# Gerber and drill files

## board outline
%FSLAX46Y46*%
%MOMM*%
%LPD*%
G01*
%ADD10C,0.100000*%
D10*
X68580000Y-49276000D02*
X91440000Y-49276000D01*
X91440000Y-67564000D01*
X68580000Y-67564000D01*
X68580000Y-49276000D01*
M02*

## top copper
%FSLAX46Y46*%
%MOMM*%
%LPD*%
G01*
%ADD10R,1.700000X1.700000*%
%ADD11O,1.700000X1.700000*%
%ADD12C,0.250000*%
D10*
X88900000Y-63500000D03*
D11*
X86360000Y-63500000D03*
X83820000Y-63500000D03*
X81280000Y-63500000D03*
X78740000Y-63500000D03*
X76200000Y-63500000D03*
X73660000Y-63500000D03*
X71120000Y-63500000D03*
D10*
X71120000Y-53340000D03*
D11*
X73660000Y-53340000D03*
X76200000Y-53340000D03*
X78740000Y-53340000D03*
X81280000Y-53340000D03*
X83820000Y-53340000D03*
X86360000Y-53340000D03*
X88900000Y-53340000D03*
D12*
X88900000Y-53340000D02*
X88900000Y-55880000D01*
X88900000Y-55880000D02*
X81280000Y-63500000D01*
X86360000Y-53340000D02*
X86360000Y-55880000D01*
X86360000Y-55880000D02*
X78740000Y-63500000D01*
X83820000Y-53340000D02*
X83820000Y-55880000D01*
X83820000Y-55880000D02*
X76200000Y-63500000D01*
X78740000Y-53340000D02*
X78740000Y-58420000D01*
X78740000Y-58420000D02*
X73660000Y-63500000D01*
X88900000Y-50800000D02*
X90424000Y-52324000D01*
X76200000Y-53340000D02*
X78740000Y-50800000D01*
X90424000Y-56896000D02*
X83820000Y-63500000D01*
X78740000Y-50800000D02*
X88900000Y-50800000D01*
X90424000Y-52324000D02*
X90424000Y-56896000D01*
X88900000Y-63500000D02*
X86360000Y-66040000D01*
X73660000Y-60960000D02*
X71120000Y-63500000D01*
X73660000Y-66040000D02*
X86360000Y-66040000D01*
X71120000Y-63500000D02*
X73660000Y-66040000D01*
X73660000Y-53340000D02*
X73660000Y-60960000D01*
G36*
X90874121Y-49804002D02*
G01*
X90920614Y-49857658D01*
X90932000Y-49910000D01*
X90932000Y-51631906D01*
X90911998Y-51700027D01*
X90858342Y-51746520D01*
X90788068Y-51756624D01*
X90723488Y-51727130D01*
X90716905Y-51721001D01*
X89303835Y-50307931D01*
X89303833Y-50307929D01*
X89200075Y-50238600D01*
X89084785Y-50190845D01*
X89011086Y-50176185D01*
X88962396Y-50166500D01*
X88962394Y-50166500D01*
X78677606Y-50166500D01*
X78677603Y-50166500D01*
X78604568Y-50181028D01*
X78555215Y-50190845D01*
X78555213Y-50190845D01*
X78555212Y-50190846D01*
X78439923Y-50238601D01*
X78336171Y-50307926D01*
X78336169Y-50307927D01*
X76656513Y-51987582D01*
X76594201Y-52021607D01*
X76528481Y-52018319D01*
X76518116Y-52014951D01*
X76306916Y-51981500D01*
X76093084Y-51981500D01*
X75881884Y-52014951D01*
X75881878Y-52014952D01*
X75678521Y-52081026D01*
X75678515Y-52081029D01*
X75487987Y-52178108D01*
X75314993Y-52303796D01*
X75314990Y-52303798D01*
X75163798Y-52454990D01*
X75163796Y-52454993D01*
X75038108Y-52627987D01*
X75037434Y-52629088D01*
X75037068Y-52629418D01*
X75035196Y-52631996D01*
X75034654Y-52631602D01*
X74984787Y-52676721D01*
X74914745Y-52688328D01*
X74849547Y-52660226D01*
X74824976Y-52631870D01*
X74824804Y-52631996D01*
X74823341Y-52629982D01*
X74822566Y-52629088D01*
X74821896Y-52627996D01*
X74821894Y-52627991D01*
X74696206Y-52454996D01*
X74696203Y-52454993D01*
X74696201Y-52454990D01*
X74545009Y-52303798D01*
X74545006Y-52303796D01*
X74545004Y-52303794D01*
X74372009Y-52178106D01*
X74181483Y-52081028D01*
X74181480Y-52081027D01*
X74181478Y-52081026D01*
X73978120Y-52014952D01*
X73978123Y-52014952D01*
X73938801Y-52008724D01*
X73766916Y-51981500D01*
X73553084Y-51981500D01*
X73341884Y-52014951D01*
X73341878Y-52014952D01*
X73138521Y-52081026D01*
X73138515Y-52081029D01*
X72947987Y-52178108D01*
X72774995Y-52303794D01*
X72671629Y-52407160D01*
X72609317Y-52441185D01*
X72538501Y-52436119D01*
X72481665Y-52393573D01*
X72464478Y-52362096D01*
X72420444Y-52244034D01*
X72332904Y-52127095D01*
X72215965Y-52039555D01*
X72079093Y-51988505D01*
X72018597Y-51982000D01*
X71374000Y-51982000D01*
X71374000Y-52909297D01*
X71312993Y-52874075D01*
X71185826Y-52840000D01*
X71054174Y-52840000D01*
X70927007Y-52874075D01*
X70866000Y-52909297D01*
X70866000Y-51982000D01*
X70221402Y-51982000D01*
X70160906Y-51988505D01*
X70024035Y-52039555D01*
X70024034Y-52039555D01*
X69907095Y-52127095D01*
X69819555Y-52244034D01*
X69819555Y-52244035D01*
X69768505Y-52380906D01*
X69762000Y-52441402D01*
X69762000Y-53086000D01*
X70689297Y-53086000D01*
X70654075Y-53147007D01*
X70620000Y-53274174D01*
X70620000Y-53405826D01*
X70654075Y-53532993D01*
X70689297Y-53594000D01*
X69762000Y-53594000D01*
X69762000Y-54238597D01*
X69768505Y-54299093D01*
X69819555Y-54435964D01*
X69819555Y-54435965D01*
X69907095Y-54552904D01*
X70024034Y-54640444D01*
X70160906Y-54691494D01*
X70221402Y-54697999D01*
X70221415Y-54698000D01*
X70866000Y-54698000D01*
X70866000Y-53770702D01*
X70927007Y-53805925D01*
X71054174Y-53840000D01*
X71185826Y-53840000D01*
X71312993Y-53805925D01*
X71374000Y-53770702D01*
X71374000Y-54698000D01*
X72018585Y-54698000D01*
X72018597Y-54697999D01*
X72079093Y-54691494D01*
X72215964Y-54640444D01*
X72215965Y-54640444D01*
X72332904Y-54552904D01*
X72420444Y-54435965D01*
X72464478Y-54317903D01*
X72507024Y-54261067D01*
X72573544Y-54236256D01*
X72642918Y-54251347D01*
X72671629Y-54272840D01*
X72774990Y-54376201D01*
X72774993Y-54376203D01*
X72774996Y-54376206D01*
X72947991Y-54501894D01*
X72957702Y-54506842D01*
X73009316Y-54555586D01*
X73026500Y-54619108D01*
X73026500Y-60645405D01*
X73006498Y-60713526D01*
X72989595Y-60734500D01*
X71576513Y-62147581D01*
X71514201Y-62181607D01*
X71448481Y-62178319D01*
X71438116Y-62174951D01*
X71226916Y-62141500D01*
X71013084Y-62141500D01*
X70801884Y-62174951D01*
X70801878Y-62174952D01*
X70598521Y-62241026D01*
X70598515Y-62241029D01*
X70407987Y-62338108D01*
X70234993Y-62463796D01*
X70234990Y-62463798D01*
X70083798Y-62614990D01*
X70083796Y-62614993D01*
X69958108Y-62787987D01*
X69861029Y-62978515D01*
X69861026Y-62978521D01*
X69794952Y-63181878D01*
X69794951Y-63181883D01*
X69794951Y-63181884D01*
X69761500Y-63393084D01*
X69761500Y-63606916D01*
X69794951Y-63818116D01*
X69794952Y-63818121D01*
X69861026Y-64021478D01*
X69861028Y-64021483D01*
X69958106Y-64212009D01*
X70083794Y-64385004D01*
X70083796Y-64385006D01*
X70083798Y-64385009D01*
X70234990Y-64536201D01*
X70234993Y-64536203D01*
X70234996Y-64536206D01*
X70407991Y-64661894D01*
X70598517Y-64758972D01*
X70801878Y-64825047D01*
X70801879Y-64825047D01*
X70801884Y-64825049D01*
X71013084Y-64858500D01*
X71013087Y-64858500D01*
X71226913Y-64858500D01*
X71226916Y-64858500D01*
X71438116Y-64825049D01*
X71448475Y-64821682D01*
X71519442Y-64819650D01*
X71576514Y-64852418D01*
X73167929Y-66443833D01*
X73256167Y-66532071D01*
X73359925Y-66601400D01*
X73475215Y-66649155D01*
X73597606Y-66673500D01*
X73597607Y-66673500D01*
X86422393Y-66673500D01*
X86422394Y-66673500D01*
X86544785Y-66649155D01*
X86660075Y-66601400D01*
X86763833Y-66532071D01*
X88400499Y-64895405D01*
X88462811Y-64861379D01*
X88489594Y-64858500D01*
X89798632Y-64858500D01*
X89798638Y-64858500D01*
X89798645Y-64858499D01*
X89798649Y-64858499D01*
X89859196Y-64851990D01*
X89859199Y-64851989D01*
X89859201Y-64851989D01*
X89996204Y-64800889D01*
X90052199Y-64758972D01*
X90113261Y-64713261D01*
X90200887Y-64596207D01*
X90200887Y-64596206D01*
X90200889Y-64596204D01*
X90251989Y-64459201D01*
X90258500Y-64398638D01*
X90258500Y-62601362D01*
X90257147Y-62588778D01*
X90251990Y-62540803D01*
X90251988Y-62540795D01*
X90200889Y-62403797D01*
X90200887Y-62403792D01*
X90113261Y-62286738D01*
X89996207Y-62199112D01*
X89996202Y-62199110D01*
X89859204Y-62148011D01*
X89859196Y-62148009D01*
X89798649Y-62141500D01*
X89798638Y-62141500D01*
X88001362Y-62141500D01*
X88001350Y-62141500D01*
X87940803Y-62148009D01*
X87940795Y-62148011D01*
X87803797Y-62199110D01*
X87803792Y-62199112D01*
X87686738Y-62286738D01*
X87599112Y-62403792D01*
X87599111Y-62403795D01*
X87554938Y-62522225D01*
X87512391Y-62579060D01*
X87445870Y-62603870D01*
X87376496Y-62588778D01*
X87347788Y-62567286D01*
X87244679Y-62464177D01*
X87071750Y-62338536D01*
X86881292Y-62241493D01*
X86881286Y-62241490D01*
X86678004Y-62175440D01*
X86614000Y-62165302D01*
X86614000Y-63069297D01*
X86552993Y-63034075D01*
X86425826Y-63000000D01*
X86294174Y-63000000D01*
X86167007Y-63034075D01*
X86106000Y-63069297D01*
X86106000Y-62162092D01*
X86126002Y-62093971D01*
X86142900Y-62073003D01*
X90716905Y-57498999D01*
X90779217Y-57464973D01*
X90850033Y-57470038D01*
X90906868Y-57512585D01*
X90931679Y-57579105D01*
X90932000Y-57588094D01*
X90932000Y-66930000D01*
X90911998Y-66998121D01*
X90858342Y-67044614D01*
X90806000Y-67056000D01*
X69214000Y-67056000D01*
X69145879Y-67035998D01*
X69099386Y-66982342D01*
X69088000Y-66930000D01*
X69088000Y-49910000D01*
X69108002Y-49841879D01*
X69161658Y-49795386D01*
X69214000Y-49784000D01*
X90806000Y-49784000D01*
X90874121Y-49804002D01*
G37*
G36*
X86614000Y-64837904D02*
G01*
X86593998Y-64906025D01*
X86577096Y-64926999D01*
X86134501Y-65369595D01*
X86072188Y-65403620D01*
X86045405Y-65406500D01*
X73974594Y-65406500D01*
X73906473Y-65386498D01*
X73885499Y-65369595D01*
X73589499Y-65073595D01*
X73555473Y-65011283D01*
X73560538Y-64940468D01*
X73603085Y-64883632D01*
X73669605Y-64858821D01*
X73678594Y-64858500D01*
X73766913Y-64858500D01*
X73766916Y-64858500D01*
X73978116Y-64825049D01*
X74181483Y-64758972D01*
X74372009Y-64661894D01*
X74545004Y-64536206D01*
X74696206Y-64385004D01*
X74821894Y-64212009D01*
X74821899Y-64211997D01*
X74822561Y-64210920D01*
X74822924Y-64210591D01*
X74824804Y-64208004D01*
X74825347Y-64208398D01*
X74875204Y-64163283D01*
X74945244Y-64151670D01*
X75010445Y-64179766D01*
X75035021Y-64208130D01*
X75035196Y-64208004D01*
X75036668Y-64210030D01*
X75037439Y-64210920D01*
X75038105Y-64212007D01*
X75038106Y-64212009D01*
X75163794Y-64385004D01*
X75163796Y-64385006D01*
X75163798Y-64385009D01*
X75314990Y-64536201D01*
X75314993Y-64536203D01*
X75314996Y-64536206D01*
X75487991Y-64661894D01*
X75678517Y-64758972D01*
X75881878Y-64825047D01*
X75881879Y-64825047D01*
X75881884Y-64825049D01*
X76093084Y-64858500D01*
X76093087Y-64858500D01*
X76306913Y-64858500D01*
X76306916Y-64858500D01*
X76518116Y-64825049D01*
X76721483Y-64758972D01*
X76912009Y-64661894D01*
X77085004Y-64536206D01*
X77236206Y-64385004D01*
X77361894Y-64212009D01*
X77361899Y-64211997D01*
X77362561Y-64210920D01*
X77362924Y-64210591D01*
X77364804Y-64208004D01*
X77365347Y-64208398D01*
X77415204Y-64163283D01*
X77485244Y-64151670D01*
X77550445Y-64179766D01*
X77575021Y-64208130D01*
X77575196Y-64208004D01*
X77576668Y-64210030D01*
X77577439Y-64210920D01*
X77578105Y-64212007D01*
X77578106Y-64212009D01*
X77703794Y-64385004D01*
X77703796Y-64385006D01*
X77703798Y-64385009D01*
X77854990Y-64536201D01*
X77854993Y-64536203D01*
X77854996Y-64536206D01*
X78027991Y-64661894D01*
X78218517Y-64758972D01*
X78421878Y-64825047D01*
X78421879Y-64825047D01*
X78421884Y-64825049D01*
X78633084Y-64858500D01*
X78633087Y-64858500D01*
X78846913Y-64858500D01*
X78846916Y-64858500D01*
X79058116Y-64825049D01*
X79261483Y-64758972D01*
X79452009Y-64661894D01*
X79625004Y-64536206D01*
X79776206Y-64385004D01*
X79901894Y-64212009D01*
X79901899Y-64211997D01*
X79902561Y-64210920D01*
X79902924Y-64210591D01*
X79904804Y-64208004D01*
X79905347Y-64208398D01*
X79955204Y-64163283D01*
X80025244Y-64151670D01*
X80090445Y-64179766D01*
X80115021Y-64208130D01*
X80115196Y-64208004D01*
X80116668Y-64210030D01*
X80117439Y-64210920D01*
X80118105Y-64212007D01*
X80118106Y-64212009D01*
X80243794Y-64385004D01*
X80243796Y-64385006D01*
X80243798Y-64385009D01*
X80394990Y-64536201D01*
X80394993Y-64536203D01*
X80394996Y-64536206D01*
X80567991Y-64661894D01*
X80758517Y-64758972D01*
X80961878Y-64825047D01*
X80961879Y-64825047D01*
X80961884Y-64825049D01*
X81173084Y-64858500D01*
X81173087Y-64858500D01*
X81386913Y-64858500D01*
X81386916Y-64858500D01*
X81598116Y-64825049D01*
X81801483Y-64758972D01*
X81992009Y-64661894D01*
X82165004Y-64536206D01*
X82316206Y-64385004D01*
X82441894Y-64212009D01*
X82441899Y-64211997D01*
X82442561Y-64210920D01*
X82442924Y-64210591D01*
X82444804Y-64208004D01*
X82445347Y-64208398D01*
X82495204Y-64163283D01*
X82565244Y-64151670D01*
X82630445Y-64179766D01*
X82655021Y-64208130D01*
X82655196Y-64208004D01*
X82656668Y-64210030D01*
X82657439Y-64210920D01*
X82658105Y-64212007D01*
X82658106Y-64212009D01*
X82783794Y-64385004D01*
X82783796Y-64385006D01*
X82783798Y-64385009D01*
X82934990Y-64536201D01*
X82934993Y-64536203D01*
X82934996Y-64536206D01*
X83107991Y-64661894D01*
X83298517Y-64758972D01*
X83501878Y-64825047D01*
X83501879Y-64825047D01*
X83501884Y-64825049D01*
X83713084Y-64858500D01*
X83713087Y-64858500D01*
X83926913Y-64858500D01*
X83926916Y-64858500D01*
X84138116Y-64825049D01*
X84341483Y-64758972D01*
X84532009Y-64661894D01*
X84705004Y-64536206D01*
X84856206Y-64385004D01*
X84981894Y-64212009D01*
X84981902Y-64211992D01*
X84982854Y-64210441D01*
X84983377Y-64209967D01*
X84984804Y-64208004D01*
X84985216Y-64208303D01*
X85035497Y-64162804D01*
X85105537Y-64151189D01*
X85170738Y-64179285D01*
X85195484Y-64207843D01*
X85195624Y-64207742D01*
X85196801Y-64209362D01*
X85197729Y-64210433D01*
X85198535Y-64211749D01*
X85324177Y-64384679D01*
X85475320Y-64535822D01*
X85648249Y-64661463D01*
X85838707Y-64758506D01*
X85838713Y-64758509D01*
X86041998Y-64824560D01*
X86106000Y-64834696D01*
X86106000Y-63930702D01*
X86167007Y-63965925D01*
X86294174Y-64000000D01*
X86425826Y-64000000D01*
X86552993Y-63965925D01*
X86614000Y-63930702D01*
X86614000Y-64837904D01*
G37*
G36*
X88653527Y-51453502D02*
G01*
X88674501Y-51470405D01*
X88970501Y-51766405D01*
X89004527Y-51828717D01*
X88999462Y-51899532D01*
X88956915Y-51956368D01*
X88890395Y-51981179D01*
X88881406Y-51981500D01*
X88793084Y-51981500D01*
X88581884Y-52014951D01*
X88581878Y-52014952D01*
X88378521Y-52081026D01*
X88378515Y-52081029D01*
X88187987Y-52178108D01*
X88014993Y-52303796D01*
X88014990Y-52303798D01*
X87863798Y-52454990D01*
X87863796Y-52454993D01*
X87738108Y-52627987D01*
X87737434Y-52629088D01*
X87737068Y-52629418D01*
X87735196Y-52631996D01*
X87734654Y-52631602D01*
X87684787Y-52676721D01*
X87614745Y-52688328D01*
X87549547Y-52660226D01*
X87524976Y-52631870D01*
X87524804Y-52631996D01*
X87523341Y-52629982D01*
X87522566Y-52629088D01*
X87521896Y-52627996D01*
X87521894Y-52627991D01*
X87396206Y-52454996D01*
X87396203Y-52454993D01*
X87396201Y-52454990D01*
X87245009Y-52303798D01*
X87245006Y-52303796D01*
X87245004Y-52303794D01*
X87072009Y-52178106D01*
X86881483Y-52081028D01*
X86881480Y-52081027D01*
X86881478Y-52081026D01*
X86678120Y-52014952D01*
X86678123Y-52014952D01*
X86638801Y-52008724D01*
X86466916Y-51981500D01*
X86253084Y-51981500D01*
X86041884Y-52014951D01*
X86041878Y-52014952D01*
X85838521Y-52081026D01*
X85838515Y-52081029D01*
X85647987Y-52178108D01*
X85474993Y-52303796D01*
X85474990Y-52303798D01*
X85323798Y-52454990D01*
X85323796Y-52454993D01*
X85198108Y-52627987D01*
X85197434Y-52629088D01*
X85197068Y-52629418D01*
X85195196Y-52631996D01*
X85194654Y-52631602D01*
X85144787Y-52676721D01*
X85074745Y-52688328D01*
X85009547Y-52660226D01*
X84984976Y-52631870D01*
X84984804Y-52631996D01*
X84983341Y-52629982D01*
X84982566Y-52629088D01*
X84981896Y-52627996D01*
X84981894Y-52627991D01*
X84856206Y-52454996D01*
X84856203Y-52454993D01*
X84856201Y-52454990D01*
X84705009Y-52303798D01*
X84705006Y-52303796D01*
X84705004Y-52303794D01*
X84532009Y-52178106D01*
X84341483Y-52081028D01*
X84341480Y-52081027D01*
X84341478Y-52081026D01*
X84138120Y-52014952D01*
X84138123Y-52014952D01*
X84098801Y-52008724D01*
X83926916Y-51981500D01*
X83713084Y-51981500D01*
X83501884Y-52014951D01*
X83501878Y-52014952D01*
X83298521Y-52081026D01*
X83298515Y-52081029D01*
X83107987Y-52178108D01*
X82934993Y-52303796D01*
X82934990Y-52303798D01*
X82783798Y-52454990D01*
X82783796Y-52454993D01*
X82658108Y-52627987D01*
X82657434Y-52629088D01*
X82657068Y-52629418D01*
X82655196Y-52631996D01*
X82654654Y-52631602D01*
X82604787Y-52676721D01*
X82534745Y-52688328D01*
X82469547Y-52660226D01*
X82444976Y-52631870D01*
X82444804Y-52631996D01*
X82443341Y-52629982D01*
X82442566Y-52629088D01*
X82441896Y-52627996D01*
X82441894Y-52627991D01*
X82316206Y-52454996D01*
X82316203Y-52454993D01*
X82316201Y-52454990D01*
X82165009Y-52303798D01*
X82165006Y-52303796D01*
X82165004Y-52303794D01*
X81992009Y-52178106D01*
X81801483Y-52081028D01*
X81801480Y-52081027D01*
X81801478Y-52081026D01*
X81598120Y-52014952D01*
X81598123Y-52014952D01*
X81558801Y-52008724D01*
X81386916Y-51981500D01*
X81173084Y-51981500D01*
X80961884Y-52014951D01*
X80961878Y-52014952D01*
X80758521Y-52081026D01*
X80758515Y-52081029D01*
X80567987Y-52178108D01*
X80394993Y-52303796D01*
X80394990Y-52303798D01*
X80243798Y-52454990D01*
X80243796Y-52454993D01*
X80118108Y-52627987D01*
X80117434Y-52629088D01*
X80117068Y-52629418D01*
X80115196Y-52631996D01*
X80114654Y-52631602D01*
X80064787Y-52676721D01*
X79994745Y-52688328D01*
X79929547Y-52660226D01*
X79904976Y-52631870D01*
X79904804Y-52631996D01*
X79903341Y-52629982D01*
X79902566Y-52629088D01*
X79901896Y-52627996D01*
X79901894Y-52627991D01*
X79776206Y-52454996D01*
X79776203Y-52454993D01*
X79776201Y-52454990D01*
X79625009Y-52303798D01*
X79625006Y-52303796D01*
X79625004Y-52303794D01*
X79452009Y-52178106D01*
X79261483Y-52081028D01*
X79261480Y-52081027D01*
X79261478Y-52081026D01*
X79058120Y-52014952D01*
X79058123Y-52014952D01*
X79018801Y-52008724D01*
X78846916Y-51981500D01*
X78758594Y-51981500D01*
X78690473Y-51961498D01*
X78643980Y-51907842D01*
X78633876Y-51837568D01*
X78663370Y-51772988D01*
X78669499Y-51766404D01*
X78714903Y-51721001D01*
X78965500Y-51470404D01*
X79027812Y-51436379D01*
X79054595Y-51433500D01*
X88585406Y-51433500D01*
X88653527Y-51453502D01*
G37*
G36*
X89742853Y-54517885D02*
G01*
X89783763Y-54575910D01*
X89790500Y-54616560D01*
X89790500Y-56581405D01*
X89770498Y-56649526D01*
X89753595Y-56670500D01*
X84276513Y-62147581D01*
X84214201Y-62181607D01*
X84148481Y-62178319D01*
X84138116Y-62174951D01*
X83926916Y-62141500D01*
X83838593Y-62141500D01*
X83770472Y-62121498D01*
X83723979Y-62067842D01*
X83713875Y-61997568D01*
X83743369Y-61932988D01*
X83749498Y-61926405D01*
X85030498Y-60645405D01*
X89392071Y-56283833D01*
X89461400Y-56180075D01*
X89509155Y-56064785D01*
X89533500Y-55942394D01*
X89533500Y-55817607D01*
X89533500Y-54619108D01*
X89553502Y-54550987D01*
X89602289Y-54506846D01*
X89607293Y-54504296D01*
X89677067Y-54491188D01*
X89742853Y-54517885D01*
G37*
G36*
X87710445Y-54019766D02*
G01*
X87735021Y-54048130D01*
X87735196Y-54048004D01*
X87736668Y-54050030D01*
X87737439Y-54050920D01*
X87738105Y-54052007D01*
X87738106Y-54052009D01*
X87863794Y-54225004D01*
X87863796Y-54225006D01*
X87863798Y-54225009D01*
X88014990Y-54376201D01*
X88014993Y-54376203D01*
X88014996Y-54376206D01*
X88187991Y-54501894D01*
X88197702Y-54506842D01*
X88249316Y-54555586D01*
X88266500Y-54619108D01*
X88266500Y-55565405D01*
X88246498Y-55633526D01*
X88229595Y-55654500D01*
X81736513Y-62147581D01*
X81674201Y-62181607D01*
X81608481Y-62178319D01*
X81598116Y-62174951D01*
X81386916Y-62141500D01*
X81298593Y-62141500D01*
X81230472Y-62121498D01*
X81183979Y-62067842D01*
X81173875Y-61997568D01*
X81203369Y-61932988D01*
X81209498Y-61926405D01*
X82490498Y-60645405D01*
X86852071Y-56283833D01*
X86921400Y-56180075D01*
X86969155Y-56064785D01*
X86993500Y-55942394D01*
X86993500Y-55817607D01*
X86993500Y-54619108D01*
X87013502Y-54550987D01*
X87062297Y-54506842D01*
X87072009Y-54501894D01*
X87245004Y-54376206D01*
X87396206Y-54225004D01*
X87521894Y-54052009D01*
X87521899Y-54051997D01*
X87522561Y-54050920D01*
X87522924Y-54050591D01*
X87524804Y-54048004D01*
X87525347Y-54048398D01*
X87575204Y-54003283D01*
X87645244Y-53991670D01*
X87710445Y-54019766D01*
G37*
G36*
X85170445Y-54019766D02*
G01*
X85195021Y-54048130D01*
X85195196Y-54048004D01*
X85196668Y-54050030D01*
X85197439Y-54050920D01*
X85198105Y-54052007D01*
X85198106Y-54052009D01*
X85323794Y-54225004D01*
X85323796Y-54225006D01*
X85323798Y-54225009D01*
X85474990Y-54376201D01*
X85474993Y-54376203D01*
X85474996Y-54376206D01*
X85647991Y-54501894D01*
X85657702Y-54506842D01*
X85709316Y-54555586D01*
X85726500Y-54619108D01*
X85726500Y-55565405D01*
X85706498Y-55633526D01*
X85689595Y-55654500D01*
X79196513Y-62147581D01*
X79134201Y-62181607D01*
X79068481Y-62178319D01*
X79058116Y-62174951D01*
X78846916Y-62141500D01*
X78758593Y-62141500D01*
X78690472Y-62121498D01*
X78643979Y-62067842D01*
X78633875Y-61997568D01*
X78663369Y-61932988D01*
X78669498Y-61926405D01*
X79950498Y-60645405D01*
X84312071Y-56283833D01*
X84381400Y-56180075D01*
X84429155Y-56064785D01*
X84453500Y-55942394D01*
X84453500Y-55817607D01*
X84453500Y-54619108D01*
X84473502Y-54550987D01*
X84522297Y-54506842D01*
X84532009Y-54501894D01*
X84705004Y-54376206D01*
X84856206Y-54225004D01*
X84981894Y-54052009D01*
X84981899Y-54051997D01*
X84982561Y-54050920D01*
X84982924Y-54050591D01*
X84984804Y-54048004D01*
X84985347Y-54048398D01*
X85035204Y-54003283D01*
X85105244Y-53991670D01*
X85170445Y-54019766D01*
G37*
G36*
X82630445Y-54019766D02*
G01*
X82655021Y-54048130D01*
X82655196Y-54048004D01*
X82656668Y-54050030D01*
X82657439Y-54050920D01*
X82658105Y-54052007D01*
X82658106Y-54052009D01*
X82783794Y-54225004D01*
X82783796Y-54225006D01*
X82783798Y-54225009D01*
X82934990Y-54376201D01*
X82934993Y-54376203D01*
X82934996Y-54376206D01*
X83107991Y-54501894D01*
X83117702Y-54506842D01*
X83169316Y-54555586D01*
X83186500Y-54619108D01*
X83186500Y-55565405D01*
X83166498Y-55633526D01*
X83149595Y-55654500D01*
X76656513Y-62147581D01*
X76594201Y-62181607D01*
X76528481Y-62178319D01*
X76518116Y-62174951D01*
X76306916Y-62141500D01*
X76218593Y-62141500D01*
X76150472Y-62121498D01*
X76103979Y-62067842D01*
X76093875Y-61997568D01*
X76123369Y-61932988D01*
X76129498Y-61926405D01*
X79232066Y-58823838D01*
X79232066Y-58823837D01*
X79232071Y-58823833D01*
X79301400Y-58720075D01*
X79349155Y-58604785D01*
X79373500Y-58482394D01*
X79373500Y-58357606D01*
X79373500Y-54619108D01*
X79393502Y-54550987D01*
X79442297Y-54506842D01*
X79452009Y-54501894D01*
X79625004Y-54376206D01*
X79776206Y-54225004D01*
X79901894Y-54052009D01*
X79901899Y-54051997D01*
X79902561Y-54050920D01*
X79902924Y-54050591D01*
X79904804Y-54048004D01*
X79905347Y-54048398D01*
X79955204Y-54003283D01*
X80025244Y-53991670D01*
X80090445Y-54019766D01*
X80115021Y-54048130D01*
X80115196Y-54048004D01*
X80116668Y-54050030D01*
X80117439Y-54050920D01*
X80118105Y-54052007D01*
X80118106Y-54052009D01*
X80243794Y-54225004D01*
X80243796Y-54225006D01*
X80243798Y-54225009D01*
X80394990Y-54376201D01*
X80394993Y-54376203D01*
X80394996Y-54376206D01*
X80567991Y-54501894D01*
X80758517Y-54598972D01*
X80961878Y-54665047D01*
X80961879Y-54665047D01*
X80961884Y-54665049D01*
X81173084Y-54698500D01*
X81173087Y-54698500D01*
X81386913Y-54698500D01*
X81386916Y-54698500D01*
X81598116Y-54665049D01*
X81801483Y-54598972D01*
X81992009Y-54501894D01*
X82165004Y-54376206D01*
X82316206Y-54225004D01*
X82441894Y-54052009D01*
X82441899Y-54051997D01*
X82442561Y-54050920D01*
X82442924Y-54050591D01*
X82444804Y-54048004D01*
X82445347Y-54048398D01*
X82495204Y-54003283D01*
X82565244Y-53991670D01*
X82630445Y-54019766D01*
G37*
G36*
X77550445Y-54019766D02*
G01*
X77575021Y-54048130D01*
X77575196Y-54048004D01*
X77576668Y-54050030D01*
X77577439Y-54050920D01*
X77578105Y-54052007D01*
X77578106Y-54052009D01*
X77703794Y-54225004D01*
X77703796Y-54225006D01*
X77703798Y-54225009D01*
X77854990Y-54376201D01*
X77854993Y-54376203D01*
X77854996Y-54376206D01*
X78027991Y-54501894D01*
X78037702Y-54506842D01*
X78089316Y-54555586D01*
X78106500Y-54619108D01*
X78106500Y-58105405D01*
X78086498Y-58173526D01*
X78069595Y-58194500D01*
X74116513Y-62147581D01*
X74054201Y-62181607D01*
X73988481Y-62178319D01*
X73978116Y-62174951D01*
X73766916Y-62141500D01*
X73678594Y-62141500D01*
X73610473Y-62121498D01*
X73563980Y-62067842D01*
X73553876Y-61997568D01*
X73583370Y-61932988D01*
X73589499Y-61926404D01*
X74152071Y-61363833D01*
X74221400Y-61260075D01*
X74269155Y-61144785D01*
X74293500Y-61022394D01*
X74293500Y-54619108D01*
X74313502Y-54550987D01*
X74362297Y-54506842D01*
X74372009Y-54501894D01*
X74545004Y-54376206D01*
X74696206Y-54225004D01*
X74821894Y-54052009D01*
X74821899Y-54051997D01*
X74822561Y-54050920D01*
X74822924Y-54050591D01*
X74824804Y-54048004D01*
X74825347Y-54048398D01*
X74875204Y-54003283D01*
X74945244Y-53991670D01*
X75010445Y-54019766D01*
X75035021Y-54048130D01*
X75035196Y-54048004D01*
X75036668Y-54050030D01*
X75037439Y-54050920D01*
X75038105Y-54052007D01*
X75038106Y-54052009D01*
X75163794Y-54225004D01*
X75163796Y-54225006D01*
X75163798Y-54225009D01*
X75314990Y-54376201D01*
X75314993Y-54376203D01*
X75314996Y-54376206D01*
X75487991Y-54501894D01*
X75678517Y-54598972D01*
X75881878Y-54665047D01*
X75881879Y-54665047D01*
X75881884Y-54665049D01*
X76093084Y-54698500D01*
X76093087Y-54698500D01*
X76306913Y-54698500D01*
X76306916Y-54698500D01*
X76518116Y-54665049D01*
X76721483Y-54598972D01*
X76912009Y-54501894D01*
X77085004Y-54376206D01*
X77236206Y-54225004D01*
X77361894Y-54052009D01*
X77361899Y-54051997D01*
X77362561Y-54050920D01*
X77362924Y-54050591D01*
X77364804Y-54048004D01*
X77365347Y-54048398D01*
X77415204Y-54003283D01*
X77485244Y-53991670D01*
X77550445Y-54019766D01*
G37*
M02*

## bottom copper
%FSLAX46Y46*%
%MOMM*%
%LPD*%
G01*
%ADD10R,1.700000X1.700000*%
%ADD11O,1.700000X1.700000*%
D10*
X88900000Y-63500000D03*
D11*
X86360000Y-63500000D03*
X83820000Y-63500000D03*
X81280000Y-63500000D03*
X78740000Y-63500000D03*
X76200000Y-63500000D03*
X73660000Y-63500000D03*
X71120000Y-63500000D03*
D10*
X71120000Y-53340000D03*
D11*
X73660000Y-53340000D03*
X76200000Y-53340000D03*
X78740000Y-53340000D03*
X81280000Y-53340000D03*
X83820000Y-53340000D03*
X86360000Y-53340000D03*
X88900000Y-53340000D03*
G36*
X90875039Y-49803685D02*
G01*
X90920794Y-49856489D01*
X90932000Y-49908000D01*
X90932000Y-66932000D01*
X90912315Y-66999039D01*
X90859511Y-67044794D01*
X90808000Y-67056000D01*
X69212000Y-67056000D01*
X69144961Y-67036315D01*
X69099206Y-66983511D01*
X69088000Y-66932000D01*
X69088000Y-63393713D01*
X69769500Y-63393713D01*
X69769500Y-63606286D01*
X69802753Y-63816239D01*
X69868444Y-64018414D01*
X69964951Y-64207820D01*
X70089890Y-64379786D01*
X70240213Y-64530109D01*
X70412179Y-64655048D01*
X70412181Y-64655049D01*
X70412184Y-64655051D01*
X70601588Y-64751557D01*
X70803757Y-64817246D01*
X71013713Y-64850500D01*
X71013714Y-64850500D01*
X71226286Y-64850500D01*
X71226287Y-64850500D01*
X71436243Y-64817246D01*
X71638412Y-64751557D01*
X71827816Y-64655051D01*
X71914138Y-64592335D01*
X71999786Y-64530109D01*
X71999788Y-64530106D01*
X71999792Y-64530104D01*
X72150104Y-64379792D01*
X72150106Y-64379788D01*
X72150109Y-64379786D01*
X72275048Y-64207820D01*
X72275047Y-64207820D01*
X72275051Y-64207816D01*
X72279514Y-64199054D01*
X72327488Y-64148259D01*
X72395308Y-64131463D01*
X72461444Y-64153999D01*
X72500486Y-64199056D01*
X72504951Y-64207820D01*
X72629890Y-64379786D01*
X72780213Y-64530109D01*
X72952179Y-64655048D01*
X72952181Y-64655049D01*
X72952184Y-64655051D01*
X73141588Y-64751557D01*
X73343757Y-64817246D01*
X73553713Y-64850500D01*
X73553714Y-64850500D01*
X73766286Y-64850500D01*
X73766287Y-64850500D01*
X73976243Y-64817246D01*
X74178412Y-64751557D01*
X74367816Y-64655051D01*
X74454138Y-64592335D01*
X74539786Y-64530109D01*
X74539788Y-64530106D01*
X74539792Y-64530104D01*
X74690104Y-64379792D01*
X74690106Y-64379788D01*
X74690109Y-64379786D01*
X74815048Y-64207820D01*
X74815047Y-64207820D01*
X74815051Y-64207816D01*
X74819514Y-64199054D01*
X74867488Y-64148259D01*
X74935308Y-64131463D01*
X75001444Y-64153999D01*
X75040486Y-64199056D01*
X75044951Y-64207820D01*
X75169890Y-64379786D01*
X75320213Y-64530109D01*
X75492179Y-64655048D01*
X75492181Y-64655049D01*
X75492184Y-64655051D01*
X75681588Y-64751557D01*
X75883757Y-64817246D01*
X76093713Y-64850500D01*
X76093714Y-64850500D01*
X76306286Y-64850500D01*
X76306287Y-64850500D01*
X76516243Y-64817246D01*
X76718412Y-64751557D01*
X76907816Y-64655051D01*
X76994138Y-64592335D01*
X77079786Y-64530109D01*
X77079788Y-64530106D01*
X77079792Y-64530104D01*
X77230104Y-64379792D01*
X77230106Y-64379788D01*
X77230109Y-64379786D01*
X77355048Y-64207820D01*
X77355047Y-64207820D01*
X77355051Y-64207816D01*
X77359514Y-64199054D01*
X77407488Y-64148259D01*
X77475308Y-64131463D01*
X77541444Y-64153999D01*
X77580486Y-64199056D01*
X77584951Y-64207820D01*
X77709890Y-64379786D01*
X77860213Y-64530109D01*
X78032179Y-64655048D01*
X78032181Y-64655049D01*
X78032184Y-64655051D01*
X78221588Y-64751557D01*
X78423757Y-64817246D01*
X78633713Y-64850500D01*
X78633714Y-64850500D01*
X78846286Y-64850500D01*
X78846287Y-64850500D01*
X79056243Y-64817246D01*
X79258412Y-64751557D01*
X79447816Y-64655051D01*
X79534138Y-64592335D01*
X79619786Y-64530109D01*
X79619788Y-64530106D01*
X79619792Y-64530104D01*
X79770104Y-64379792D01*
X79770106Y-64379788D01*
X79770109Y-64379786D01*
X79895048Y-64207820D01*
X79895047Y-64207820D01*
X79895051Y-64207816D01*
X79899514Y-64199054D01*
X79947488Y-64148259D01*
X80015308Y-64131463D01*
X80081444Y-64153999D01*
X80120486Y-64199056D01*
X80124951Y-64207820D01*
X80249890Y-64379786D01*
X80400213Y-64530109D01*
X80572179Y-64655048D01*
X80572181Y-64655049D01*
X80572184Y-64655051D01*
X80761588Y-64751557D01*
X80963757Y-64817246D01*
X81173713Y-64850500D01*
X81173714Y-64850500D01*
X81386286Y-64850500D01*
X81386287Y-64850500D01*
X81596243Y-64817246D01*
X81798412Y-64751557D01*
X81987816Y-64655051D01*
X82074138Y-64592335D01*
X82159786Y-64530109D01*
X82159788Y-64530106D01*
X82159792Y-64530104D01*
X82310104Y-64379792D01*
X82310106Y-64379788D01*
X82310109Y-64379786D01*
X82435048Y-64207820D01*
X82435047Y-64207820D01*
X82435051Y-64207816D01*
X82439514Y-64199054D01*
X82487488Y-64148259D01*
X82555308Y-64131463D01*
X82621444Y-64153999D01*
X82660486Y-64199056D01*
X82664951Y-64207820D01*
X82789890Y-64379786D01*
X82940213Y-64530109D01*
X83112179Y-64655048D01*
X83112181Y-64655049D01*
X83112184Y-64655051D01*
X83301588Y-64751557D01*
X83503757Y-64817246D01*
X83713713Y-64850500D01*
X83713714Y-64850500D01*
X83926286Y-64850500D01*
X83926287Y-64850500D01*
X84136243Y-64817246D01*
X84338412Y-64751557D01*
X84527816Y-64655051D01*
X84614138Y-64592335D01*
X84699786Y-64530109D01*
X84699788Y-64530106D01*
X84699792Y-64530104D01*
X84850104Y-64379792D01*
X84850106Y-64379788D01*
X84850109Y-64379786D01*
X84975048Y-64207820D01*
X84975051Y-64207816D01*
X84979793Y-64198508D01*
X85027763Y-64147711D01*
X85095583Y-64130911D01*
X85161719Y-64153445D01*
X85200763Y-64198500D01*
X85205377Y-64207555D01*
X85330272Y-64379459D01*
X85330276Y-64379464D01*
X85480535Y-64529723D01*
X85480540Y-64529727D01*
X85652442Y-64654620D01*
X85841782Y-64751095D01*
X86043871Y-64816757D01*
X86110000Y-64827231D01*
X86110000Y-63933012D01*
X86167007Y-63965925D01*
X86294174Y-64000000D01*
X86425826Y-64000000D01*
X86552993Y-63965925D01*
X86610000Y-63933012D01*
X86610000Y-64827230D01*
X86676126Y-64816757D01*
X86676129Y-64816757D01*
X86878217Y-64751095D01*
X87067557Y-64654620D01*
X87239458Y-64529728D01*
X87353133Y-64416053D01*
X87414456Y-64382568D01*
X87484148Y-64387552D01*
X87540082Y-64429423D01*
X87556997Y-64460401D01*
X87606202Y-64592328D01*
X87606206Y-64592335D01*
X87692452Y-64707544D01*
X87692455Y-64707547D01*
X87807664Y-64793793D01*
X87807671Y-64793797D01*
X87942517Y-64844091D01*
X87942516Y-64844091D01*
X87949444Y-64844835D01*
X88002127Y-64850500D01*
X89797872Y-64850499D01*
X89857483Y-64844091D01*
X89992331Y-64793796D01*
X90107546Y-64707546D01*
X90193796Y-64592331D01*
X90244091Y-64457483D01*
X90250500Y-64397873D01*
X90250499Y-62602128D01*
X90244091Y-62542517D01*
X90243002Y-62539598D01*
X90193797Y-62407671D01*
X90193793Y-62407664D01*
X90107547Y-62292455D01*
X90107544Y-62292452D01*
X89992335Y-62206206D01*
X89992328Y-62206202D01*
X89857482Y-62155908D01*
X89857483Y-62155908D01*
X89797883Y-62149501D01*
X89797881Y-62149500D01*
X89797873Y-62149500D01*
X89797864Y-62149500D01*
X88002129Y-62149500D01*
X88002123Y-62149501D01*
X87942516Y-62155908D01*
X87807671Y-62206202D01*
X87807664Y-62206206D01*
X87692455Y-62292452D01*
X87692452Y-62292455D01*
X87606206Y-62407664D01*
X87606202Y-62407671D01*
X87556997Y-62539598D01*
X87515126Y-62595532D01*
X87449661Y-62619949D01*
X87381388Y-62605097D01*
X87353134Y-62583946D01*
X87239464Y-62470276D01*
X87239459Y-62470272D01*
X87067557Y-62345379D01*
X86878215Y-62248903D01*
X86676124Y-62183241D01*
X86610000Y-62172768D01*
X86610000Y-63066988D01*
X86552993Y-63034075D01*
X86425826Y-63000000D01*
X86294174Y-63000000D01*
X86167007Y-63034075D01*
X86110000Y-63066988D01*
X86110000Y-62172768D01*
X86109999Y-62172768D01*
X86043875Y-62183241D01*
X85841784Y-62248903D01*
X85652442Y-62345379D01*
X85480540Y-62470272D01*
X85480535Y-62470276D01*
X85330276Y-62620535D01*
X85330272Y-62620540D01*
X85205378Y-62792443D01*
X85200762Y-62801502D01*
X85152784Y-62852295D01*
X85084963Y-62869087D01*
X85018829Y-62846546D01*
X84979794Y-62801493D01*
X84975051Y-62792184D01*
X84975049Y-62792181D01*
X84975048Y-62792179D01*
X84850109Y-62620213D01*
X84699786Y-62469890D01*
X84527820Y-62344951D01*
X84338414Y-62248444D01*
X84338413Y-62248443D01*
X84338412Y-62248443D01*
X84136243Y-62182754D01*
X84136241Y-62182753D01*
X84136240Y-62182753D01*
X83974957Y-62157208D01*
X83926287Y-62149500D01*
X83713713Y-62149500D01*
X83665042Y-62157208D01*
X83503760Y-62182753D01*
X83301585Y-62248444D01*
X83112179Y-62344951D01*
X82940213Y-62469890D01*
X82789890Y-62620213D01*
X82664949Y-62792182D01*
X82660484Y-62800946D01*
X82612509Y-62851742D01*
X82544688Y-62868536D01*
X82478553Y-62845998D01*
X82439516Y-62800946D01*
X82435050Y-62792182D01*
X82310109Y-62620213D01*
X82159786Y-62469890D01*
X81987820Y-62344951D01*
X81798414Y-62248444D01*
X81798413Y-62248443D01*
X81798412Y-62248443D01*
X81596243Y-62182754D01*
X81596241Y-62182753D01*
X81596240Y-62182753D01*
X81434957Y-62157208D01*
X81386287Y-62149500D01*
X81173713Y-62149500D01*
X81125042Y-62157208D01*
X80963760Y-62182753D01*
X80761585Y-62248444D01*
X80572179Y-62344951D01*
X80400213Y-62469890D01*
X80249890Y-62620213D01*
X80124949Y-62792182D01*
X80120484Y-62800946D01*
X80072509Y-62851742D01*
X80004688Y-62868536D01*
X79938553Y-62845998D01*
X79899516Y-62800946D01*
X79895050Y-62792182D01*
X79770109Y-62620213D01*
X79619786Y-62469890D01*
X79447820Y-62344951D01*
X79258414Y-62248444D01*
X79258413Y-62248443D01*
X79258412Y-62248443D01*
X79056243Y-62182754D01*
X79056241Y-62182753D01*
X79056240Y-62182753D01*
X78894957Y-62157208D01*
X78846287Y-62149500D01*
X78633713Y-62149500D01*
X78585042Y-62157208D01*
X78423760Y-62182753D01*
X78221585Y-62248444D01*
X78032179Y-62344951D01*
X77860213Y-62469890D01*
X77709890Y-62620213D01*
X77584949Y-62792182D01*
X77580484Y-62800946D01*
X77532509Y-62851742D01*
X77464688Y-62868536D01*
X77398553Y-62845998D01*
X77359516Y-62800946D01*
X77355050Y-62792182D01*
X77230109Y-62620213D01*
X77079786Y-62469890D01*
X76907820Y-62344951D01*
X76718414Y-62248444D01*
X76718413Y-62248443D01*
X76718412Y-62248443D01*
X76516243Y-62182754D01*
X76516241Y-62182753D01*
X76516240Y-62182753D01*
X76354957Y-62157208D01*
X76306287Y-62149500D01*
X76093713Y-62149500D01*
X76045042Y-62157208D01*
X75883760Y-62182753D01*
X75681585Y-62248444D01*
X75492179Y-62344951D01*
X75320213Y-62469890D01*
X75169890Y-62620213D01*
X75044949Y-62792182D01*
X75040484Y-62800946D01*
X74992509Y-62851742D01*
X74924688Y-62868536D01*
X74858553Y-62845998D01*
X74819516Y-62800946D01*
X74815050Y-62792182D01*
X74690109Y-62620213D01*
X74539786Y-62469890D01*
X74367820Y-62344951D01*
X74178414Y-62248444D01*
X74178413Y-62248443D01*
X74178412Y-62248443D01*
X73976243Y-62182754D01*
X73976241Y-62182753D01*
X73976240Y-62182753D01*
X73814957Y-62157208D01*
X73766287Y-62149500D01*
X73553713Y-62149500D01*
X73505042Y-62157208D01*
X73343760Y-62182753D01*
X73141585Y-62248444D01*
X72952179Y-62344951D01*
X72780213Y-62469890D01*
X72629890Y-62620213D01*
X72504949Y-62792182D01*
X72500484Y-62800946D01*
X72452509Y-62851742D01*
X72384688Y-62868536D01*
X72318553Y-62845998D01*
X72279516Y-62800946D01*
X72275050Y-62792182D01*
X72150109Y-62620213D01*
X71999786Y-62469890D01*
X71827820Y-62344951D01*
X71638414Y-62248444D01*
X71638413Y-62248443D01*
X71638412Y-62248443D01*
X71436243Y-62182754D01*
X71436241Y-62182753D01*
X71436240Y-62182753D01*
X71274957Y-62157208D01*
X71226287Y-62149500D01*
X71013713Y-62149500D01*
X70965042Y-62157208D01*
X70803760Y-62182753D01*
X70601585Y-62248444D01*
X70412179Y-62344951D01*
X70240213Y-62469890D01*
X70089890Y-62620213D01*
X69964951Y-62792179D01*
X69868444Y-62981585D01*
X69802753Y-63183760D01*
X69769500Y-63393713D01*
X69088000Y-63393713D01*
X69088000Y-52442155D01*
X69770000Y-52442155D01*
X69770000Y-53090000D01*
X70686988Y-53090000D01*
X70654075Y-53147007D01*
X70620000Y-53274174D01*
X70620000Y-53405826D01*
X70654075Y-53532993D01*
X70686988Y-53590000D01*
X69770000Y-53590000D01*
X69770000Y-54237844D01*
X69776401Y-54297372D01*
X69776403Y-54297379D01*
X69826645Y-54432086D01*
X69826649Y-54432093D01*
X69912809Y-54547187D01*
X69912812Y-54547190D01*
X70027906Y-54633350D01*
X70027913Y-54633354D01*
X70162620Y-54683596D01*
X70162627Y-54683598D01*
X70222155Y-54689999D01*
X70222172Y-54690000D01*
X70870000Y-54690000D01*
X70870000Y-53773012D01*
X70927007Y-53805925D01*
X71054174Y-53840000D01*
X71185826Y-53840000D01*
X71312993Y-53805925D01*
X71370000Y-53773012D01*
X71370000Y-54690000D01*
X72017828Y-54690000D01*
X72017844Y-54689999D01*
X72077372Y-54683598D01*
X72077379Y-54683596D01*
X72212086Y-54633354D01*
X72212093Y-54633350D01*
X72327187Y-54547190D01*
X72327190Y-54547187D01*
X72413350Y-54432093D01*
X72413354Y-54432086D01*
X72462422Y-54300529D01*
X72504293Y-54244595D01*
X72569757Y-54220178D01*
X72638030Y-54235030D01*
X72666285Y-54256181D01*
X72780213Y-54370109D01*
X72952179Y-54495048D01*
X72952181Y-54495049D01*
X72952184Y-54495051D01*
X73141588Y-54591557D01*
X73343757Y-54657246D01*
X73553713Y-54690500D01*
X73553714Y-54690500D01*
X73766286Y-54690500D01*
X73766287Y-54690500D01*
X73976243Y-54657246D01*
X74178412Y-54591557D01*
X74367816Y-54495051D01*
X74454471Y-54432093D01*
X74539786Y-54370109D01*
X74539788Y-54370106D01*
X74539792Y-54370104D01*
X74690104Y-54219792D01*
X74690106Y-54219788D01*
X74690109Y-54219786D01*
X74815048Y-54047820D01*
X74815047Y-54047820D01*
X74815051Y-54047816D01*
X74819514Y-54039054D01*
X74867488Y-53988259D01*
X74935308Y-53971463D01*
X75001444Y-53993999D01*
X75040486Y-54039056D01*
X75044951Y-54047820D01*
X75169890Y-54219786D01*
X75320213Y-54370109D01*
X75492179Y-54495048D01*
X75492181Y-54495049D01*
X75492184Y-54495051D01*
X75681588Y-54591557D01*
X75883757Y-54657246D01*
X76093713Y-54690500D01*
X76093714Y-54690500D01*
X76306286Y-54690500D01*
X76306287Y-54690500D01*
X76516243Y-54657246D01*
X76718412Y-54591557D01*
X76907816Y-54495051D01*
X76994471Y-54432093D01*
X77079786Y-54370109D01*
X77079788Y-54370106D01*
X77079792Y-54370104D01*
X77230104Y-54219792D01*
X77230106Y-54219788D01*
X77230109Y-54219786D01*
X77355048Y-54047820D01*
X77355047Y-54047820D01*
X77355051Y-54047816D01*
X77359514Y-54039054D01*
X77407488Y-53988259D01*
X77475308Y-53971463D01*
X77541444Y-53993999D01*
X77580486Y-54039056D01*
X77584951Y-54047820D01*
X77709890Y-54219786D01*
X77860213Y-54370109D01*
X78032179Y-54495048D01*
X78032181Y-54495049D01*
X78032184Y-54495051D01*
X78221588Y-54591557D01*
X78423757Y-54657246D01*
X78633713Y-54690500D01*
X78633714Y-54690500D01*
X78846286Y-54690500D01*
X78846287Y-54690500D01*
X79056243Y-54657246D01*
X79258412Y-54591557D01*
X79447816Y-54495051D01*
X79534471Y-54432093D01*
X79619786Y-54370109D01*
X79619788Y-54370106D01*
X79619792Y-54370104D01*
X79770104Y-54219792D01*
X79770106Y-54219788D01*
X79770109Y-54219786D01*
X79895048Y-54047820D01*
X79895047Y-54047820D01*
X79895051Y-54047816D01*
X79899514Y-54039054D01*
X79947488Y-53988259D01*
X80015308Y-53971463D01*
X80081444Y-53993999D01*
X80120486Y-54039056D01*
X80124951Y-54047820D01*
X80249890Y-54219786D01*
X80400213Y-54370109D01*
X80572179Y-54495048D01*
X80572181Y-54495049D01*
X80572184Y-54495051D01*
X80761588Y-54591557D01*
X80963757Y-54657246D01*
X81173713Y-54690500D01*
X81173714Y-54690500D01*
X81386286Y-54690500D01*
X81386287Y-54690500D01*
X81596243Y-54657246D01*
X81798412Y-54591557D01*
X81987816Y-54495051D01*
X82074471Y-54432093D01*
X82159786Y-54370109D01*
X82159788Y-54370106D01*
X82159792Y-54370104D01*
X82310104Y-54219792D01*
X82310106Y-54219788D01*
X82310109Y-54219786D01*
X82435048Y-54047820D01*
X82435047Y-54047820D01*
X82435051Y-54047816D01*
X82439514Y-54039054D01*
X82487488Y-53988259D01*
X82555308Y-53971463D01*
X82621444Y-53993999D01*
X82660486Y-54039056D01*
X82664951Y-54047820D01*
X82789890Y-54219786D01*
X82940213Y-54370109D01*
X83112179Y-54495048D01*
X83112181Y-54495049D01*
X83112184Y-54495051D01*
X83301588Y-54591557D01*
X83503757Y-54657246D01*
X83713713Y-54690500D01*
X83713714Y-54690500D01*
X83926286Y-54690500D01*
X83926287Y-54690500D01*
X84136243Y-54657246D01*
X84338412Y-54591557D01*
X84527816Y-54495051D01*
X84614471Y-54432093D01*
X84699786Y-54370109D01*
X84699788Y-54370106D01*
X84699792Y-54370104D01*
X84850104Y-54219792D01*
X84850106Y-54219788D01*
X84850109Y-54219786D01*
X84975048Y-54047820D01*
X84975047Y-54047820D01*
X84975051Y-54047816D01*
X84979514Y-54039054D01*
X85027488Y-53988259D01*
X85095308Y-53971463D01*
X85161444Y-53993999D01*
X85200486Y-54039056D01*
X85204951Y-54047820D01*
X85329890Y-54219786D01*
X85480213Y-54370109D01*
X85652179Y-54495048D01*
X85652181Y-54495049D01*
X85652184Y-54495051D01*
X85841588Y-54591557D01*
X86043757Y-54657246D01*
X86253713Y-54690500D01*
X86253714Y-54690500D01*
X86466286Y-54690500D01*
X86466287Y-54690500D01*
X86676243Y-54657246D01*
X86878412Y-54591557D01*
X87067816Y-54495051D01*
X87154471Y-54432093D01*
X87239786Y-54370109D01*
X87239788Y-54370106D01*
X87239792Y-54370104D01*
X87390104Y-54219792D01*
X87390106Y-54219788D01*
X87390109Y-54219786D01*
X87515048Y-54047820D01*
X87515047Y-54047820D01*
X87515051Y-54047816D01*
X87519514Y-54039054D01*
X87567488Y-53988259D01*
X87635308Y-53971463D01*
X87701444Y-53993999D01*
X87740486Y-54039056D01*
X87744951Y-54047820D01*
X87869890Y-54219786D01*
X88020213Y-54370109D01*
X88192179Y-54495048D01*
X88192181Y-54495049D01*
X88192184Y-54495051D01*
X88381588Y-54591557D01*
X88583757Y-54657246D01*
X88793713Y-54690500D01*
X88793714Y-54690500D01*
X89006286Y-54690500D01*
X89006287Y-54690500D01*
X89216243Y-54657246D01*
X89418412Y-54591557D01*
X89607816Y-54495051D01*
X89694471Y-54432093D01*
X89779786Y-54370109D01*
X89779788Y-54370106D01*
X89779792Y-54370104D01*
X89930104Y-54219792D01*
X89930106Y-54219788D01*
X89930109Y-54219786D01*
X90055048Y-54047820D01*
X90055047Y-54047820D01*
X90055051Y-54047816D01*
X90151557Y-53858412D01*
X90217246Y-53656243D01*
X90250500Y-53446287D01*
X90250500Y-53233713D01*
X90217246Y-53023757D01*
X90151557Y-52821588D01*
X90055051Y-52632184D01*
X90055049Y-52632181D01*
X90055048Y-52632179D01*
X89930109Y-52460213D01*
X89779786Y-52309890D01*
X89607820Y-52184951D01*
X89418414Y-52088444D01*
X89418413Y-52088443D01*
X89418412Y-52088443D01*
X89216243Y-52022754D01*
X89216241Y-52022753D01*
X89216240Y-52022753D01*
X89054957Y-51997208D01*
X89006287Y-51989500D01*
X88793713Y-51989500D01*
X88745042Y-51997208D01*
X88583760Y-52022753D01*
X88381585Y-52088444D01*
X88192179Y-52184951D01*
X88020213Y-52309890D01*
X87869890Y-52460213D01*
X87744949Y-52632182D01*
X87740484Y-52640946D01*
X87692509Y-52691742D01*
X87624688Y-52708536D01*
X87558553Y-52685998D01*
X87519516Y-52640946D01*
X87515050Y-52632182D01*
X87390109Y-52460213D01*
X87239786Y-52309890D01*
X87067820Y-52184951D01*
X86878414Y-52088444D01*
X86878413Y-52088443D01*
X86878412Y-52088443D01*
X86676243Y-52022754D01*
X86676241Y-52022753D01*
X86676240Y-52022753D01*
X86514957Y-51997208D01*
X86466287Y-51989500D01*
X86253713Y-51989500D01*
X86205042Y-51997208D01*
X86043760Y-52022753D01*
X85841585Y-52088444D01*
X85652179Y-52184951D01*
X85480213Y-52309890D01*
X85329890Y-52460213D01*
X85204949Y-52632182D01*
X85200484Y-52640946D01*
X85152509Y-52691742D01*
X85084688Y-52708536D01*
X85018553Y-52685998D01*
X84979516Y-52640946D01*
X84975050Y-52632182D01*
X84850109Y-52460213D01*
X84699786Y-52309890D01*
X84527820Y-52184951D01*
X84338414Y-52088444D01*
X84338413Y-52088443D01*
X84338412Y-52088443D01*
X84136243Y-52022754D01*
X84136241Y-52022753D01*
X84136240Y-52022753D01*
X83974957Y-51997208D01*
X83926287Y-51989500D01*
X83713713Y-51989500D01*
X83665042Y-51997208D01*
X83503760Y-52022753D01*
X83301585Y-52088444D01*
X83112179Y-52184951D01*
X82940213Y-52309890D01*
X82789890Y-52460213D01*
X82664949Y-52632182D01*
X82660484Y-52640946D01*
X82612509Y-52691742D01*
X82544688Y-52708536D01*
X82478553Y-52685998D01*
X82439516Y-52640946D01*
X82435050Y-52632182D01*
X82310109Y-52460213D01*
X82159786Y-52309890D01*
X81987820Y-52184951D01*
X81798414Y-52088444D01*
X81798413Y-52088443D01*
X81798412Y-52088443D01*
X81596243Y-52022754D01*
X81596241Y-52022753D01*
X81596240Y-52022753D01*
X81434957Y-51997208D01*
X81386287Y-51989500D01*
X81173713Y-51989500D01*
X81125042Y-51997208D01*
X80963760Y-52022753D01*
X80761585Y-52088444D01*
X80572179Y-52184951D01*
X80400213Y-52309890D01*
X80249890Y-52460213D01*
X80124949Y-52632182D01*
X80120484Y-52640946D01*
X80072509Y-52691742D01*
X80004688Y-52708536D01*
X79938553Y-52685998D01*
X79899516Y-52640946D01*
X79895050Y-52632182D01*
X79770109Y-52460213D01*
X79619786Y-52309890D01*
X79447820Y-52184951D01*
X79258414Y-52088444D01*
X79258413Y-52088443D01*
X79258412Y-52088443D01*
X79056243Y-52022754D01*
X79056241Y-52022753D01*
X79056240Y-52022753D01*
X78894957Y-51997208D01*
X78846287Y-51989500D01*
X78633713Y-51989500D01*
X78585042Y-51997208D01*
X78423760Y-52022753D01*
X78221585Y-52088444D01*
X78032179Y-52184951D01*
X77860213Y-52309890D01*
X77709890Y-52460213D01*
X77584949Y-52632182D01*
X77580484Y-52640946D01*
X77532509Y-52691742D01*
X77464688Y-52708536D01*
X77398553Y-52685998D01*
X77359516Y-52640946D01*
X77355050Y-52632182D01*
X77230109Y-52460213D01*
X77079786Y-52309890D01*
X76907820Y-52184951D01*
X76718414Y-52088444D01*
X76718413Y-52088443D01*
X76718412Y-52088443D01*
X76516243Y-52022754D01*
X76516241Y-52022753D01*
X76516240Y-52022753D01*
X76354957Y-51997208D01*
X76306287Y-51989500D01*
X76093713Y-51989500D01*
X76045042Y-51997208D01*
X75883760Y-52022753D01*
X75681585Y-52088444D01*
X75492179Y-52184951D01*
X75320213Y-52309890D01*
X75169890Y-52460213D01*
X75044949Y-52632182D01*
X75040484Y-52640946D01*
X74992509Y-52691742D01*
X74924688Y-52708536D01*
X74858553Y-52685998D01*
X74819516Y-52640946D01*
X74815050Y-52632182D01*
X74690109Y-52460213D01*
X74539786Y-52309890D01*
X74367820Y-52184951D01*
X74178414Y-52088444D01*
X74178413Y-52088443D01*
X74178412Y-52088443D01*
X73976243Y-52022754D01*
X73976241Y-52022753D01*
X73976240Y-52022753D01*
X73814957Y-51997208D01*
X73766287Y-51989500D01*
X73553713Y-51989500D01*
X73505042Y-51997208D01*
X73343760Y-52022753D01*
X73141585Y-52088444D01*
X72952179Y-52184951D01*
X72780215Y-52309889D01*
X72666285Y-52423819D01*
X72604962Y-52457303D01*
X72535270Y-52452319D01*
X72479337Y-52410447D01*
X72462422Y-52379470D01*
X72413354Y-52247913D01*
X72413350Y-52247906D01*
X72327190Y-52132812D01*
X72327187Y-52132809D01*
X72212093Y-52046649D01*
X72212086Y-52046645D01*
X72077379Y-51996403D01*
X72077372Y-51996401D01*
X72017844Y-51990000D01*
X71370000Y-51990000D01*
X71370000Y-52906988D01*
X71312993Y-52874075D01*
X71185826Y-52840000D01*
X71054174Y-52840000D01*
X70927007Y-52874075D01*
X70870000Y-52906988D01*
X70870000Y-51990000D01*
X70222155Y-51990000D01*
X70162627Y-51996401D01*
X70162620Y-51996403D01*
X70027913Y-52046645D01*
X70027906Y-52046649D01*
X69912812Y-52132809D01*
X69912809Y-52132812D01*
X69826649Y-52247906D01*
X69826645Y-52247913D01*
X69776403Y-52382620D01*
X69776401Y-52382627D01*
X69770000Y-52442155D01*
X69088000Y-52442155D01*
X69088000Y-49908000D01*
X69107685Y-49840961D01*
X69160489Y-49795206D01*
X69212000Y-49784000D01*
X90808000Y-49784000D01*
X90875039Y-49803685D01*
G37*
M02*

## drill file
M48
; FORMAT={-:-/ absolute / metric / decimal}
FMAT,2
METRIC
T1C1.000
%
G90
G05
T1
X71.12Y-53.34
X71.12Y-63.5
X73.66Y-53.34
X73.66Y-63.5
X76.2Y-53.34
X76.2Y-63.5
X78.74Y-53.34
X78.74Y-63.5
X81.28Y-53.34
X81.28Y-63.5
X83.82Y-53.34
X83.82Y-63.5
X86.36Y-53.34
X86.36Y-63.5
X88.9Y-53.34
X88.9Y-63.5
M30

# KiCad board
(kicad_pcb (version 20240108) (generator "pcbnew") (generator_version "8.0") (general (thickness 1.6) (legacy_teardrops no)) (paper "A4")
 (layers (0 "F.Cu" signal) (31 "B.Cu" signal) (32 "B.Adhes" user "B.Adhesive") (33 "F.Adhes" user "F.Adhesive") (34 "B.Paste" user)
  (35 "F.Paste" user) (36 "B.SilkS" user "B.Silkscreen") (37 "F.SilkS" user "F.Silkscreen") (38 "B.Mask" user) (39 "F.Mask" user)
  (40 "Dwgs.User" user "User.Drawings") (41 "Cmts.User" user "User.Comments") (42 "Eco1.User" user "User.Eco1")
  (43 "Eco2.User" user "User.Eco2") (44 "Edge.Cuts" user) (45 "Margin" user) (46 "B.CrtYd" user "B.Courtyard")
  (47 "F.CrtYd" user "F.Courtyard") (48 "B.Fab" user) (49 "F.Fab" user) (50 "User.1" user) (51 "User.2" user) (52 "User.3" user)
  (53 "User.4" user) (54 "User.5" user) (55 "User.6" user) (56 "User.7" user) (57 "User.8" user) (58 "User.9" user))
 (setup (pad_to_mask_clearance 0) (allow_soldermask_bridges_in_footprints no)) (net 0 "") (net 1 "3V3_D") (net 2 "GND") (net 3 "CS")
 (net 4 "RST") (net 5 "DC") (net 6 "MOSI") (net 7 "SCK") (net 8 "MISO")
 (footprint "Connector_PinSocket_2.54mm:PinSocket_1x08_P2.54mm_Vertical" (layer "F.Cu") (at 88.9 63.5 -90)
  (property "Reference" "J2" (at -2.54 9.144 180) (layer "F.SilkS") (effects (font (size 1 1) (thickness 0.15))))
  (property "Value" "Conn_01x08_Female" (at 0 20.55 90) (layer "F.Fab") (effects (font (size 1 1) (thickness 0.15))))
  (pad "1" thru_hole rect (at 0 0 270) (size 1.7 1.7) (drill 1) (layers "*.Cu" "*.Mask") (remove_unused_layers no) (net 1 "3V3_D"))
  (pad "2" thru_hole oval (at 0 2.54 270) (size 1.7 1.7) (drill 1) (layers "*.Cu" "*.Mask") (remove_unused_layers no) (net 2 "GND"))
  (pad "3" thru_hole oval (at 0 5.08 270) (size 1.7 1.7) (drill 1) (layers "*.Cu" "*.Mask") (remove_unused_layers no) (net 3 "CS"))
  (pad "4" thru_hole oval (at 0 7.62 270) (size 1.7 1.7) (drill 1) (layers "*.Cu" "*.Mask") (remove_unused_layers no) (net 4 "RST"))
  (pad "5" thru_hole oval (at 0 10.16 270) (size 1.7 1.7) (drill 1) (layers "*.Cu" "*.Mask") (remove_unused_layers no) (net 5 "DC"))
  (pad "6" thru_hole oval (at 0 12.7 270) (size 1.7 1.7) (drill 1) (layers "*.Cu" "*.Mask") (remove_unused_layers no) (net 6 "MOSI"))
  (pad "7" thru_hole oval (at 0 15.24 270) (size 1.7 1.7) (drill 1) (layers "*.Cu" "*.Mask") (remove_unused_layers no) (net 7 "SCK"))
  (pad "8" thru_hole oval (at 0 17.78 270) (size 1.7 1.7) (drill 1) (layers "*.Cu" "*.Mask") (remove_unused_layers no) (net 1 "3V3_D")))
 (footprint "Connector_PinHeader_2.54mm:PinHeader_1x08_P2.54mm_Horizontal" (layer "F.Cu") (at 71.12 53.34 90)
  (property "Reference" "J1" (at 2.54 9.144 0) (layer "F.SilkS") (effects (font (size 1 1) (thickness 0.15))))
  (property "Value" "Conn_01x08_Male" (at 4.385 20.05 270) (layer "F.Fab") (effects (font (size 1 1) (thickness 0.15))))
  (pad "1" thru_hole rect (at 0 0 90) (size 1.7 1.7) (drill 1) (layers "*.Cu" "*.Mask") (remove_unused_layers no) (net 2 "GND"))
  (pad "2" thru_hole oval (at 0 2.54 90) (size 1.7 1.7) (drill 1) (layers "*.Cu" "*.Mask") (remove_unused_layers no) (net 1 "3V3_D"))
  (pad "3" thru_hole oval (at 0 5.08 90) (size 1.7 1.7) (drill 1) (layers "*.Cu" "*.Mask") (remove_unused_layers no) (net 3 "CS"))
  (pad "4" thru_hole oval (at 0 7.62 90) (size 1.7 1.7) (drill 1) (layers "*.Cu" "*.Mask") (remove_unused_layers no) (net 7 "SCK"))
  (pad "5" thru_hole oval (at 0 10.16 90) (size 1.7 1.7) (drill 1) (layers "*.Cu" "*.Mask") (remove_unused_layers no) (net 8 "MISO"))
  (pad "6" thru_hole oval (at 0 12.7 90) (size 1.7 1.7) (drill 1) (layers "*.Cu" "*.Mask") (remove_unused_layers no) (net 6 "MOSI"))
  (pad "7" thru_hole oval (at 0 15.24 90) (size 1.7 1.7) (drill 1) (layers "*.Cu" "*.Mask") (remove_unused_layers no) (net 5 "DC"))
  (pad "8" thru_hole oval (at 0 17.78 90) (size 1.7 1.7) (drill 1) (layers "*.Cu" "*.Mask") (remove_unused_layers no) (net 4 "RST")))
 (gr_rect (start 68.58 49.276) (end 91.44 67.564) (stroke (width 0.1) (type solid)) (fill none) (layer "Edge.Cuts"))
 (segment (start 88.9 53.34) (end 88.9 55.88) (width 0.25) (layer "F.Cu") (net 4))
 (segment (start 88.9 55.88) (end 81.28 63.5) (width 0.25) (layer "F.Cu") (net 4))
 (segment (start 86.36 53.34) (end 86.36 55.88) (width 0.25) (layer "F.Cu") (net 5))
 (segment (start 86.36 55.88) (end 78.74 63.5) (width 0.25) (layer "F.Cu") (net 5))
 (segment (start 83.82 53.34) (end 83.82 55.88) (width 0.25) (layer "F.Cu") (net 6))
 (segment (start 83.82 55.88) (end 76.2 63.5) (width 0.25) (layer "F.Cu") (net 6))
 (segment (start 78.74 53.34) (end 78.74 58.42) (width 0.25) (layer "F.Cu") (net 7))
 (segment (start 78.74 58.42) (end 73.66 63.5) (width 0.25) (layer "F.Cu") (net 7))
 (segment (start 88.9 50.8) (end 90.424 52.324) (width 0.25) (layer "F.Cu") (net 3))
 (segment (start 76.2 53.34) (end 78.74 50.8) (width 0.25) (layer "F.Cu") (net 3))
 (segment (start 90.424 56.896) (end 83.82 63.5) (width 0.25) (layer "F.Cu") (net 3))
 (segment (start 78.74 50.8) (end 88.9 50.8) (width 0.25) (layer "F.Cu") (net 3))
 (segment (start 90.424 52.324) (end 90.424 56.896) (width 0.25) (layer "F.Cu") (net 3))
 (segment (start 88.9 63.5) (end 86.36 66.04) (width 0.25) (layer "F.Cu") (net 1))
 (segment (start 73.66 60.96) (end 71.12 63.5) (width 0.25) (layer "F.Cu") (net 1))
 (segment (start 73.66 66.04) (end 86.36 66.04) (width 0.25) (layer "F.Cu") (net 1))
 (segment (start 71.12 63.5) (end 73.66 66.04) (width 0.25) (layer "F.Cu") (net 1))
 (segment (start 73.66 53.34) (end 73.66 60.96) (width 0.25) (layer "F.Cu") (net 1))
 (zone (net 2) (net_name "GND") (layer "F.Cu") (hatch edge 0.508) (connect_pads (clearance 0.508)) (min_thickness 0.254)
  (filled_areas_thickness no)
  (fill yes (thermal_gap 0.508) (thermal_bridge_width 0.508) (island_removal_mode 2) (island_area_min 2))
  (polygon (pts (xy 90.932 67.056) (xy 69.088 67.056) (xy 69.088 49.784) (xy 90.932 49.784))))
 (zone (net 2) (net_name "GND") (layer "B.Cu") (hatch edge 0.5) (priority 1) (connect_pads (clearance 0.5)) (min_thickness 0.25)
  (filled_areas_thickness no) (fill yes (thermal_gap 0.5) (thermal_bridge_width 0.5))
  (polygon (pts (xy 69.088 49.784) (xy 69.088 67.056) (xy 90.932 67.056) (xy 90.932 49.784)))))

